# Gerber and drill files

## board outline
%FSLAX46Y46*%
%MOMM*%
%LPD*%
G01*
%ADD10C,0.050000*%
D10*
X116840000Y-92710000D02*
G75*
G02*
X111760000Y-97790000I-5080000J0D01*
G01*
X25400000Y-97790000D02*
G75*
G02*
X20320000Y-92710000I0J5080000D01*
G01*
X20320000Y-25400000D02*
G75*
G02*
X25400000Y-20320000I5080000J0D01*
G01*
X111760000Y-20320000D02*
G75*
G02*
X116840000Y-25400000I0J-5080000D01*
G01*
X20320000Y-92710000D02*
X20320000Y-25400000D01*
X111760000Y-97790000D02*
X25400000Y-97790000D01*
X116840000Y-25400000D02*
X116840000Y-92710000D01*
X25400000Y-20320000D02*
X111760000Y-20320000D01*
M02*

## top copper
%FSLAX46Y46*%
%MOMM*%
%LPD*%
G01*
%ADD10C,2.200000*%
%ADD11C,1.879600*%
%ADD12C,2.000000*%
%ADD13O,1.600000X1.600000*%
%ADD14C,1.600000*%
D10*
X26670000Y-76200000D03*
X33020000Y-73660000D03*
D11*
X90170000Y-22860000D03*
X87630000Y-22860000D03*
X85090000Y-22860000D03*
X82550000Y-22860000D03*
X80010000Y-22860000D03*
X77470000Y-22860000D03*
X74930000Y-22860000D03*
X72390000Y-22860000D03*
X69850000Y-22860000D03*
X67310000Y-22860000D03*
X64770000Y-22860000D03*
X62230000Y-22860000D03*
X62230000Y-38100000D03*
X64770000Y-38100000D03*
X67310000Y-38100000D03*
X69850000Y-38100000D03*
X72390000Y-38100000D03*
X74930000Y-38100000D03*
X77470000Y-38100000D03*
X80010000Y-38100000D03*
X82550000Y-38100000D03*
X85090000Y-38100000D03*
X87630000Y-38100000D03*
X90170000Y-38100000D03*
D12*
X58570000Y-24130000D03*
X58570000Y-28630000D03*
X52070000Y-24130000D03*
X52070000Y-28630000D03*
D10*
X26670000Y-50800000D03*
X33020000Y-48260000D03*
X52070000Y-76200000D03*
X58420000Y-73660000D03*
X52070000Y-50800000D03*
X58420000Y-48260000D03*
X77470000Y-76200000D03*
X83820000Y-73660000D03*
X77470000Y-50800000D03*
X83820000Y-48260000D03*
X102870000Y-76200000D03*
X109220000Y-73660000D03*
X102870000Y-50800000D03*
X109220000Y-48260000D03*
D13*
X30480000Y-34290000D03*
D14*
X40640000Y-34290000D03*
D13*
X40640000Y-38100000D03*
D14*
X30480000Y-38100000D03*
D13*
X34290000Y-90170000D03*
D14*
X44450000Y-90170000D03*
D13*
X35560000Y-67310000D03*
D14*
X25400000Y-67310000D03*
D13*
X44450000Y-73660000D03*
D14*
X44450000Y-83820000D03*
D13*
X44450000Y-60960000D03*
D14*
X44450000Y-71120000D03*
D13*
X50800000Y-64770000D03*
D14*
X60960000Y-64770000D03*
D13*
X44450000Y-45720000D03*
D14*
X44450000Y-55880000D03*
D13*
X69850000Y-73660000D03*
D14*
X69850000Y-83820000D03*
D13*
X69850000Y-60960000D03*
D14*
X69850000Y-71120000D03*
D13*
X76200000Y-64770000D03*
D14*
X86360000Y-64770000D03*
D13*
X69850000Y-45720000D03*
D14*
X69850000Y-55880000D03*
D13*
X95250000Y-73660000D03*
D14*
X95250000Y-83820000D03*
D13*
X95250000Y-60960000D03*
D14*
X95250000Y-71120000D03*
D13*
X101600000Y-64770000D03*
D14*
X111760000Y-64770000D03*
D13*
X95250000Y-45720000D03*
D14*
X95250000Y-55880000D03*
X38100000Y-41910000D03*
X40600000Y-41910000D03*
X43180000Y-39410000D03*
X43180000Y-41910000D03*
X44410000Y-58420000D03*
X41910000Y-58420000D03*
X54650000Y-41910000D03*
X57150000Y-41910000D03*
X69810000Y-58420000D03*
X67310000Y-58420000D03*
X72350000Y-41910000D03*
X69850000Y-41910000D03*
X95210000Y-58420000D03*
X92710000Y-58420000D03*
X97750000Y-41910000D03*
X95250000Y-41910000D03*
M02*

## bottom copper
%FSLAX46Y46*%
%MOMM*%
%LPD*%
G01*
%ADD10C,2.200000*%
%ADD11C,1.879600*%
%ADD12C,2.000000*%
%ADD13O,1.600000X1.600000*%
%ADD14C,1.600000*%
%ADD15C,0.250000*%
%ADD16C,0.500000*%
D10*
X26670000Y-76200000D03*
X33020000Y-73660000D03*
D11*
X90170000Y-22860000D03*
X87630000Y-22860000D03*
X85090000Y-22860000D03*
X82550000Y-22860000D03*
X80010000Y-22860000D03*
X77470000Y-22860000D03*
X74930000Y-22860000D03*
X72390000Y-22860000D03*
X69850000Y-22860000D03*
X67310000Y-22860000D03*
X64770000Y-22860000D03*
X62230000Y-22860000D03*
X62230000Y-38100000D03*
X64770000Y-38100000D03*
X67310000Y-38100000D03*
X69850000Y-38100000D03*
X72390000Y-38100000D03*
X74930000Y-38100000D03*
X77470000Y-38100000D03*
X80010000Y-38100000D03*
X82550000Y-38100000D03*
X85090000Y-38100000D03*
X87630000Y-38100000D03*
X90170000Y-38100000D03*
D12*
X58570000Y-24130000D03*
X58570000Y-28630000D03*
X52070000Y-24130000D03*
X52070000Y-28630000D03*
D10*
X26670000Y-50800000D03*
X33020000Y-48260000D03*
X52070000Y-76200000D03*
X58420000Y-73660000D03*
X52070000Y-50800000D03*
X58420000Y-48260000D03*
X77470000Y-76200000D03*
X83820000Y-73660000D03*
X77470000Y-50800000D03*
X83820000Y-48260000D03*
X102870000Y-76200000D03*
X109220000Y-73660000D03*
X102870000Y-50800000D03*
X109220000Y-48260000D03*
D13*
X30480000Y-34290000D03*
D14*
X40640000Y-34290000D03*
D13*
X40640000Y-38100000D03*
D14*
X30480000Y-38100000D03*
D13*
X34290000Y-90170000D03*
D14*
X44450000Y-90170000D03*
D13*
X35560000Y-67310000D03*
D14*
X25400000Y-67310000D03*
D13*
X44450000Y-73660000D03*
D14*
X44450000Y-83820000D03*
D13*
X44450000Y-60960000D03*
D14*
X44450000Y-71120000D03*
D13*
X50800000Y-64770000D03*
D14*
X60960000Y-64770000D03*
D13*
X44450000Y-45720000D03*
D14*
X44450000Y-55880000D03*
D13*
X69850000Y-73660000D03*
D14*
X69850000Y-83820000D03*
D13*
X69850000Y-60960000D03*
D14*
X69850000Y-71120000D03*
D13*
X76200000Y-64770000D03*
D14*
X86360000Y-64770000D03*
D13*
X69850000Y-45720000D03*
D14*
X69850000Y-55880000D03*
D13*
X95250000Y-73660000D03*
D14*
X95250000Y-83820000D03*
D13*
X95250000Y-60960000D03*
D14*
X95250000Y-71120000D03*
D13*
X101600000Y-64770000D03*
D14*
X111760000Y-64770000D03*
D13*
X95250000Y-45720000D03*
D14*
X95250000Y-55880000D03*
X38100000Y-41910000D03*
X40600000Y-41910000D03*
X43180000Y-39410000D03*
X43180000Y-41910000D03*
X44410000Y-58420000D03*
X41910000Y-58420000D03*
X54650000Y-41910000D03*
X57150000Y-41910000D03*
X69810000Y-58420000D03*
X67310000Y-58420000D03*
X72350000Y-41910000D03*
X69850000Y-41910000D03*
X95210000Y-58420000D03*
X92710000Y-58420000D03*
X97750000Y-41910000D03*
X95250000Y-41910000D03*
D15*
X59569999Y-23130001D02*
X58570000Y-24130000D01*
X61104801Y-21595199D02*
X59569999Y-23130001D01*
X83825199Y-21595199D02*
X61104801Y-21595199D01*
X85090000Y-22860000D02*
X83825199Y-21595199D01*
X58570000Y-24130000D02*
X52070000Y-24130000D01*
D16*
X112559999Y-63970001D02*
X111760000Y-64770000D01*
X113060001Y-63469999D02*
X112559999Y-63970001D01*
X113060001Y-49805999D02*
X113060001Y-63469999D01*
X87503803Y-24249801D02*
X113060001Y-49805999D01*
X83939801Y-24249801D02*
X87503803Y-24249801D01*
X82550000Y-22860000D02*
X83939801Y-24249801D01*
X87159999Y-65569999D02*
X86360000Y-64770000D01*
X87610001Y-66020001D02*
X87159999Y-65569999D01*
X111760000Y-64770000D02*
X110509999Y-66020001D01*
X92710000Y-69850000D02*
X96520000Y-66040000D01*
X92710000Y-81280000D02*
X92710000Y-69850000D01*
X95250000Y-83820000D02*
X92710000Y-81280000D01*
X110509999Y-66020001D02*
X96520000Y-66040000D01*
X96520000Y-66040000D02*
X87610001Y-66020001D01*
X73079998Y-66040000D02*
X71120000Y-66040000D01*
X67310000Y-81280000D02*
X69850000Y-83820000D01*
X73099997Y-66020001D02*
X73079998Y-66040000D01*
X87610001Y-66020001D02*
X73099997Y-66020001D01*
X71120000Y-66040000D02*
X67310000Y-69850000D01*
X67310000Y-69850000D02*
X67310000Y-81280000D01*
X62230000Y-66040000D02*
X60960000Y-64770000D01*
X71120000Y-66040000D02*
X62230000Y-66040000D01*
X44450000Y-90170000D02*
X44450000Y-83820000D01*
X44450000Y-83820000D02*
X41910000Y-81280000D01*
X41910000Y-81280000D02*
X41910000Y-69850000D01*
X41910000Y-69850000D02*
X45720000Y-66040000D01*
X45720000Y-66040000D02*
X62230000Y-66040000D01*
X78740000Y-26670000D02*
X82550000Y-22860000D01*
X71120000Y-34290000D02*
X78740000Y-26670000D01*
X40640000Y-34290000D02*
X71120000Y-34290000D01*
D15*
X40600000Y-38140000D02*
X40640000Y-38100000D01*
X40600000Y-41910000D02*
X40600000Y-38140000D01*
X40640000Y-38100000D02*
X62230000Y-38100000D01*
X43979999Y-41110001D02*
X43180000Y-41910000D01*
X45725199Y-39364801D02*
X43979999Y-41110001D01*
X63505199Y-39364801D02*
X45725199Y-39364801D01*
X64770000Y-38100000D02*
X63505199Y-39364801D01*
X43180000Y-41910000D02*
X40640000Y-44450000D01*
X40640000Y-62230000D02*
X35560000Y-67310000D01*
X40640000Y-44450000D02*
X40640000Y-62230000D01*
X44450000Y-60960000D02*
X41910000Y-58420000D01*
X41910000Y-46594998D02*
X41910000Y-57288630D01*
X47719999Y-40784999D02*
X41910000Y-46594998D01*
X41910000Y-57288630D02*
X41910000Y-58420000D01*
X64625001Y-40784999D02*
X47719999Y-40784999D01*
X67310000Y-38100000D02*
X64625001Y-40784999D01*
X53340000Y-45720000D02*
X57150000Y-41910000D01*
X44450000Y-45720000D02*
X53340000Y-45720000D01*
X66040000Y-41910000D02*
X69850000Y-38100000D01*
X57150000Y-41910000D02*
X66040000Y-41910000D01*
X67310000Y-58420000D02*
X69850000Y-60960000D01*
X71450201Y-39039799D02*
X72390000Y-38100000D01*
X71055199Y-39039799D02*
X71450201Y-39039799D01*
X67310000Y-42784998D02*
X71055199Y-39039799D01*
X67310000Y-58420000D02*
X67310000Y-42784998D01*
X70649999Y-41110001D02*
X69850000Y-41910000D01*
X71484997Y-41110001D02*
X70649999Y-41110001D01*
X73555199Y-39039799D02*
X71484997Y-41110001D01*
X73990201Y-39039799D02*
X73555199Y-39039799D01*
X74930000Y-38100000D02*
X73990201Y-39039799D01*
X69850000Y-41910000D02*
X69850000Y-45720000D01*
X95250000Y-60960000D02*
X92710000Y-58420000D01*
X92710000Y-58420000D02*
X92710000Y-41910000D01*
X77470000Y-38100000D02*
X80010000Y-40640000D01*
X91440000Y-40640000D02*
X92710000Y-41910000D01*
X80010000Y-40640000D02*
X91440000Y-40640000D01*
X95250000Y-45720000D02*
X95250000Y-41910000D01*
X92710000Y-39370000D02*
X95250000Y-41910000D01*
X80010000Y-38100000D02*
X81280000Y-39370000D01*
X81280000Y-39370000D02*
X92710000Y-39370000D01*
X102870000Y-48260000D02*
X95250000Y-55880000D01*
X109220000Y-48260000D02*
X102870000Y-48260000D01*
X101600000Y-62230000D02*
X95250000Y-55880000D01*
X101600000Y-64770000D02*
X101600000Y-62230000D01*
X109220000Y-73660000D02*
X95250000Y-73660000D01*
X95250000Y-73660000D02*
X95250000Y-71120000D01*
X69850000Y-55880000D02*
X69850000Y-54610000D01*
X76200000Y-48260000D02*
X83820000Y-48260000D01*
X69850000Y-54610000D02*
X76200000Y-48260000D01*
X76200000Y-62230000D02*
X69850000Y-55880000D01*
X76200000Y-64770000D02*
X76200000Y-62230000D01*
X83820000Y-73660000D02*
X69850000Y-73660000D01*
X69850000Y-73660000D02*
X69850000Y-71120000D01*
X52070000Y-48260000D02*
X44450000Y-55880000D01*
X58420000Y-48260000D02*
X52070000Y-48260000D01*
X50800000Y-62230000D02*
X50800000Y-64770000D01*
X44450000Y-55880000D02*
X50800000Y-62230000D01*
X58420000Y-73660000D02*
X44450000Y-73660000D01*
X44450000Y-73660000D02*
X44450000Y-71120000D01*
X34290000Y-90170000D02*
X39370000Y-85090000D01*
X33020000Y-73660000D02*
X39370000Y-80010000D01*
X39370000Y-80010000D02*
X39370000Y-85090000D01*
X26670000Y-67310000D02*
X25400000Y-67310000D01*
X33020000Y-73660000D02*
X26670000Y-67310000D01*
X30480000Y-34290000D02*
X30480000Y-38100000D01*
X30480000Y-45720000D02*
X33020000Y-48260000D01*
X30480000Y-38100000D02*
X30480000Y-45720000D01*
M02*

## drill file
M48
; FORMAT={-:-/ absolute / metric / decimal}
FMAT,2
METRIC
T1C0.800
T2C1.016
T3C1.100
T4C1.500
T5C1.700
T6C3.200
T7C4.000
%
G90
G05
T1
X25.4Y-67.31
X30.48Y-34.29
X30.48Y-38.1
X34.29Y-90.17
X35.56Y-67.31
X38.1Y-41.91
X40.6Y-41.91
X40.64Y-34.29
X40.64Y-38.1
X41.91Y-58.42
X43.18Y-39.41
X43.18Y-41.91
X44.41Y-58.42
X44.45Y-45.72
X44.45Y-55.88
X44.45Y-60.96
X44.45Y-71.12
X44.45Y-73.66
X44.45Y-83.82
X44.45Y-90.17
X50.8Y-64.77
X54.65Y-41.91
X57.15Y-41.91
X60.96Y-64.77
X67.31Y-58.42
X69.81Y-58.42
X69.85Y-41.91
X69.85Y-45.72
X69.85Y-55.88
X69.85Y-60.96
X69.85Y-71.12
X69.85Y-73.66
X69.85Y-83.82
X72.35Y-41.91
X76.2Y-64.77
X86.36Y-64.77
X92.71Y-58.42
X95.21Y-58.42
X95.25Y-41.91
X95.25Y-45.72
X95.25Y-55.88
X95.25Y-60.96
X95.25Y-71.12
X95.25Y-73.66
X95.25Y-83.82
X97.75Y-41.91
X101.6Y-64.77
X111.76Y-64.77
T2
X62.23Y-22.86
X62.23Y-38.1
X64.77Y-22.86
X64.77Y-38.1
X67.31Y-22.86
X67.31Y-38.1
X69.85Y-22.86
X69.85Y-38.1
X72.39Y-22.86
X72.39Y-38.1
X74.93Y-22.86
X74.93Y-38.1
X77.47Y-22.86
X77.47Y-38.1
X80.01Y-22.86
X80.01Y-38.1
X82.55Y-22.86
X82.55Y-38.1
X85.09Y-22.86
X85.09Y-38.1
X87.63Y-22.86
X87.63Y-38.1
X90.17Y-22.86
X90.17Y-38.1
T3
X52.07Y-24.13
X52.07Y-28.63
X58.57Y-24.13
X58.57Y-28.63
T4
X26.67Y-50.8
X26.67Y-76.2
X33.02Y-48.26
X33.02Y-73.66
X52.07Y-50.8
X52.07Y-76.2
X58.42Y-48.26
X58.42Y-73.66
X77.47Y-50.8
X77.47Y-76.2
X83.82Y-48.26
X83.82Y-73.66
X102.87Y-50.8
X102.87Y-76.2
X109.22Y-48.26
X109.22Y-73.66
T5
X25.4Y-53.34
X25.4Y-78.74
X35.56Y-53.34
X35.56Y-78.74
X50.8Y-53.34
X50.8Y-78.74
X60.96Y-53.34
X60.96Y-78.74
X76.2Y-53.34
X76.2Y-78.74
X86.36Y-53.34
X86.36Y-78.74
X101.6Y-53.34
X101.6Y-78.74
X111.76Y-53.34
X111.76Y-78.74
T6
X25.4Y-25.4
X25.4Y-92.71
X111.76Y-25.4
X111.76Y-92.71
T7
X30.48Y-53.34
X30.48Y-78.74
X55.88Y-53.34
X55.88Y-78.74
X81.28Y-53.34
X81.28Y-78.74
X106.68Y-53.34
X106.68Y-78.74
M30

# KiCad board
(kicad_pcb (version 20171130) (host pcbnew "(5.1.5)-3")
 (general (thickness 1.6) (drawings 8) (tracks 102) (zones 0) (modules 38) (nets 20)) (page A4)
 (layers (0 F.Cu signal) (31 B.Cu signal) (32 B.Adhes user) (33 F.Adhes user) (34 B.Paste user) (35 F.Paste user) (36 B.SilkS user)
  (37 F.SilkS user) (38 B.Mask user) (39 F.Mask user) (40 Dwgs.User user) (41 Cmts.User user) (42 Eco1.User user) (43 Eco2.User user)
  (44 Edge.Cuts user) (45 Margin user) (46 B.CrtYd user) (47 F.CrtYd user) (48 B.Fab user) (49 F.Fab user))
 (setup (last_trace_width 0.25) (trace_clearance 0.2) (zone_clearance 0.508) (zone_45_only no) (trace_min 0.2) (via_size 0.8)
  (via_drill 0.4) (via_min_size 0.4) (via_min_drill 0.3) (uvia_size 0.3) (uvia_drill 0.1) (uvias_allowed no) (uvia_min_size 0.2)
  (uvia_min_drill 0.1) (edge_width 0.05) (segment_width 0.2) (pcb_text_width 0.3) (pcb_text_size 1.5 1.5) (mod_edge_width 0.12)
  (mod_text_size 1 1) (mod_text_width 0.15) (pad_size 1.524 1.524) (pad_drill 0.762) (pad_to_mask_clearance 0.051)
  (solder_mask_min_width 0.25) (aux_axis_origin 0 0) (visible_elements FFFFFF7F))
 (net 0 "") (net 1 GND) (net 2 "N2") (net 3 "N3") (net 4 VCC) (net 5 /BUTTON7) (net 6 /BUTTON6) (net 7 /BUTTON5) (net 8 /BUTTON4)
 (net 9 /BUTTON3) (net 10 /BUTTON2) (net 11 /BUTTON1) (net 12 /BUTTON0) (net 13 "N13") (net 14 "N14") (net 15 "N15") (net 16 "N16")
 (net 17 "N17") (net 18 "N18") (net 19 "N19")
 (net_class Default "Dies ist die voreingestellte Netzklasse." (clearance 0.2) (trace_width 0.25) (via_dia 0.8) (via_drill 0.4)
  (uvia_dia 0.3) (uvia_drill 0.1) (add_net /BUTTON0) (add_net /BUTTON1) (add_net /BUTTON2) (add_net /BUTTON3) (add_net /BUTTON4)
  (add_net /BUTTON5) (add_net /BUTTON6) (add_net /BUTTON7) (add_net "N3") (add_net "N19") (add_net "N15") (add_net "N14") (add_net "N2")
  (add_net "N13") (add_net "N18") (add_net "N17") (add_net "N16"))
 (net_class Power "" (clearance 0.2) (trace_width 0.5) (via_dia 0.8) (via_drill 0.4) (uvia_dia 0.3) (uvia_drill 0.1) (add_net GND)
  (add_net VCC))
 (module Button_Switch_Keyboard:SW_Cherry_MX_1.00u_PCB (layer F.Cu) (at 33.02 73.66)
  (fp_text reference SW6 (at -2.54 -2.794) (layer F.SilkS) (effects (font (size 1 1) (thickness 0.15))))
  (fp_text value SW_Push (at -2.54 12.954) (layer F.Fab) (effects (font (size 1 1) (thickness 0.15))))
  (pad "" np_thru_hole circle (at 2.54 5.08) (size 1.7 1.7) (drill 1.7) (layers *.Cu *.Mask))
  (pad "" np_thru_hole circle (at -7.62 5.08) (size 1.7 1.7) (drill 1.7) (layers *.Cu *.Mask))
  (pad "" np_thru_hole circle (at -2.54 5.08) (size 4 4) (drill 4) (layers *.Cu *.Mask))
  (pad 2 thru_hole circle (at -6.35 2.54) (size 2.2 2.2) (drill 1.5) (layers *.Cu *.Mask) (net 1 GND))
  (pad 1 thru_hole circle (at 0 0) (size 2.2 2.2) (drill 1.5) (layers *.Cu *.Mask) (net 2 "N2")))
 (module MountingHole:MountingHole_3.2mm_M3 (layer F.Cu) (at 25.4 25.4)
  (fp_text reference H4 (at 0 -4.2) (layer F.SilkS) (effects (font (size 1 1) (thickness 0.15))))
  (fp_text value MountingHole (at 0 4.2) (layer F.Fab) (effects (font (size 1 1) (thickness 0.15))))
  (pad 1 np_thru_hole circle (at 0 0) (size 3.2 3.2) (drill 3.2) (layers *.Cu *.Mask)))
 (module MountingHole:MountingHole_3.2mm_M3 (layer F.Cu) (at 111.76 25.4)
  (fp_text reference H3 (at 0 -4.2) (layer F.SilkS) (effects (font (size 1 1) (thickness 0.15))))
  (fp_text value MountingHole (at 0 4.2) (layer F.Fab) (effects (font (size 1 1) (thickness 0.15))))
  (pad 1 np_thru_hole circle (at 0 0) (size 3.2 3.2) (drill 3.2) (layers *.Cu *.Mask)))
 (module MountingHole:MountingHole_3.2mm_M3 (layer F.Cu) (at 111.76 92.71)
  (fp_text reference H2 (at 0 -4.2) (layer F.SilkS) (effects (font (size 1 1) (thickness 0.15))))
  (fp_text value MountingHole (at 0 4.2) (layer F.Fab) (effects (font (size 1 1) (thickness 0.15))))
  (pad 1 np_thru_hole circle (at 0 0) (size 3.2 3.2) (drill 3.2) (layers *.Cu *.Mask)))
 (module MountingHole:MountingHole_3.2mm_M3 (layer F.Cu) (at 25.4 92.71)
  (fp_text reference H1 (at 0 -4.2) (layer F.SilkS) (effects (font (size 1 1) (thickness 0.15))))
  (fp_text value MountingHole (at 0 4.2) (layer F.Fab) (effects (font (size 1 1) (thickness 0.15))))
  (pad 1 np_thru_hole circle (at 0 0) (size 3.2 3.2) (drill 3.2) (layers *.Cu *.Mask)))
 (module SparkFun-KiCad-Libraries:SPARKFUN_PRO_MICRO (layer B.Cu) (at 77.47 30.48 90)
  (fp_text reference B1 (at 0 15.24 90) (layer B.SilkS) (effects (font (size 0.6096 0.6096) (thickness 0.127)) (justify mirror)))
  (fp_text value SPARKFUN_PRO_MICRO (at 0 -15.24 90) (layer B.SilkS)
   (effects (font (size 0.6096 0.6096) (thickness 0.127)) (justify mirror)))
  (pad 24 thru_hole circle (at 7.62 12.7 90) (size 1.8796 1.8796) (drill 1.016) (layers *.Cu *.Mask) (solder_mask_margin 0.1016))
  (pad 23 thru_hole circle (at 7.62 10.16 90) (size 1.8796 1.8796) (drill 1.016) (layers *.Cu *.Mask) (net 1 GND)
   (solder_mask_margin 0.1016))
  (pad 22 thru_hole circle (at 7.62 7.62 90) (size 1.8796 1.8796) (drill 1.016) (layers *.Cu *.Mask) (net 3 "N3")
   (solder_mask_margin 0.1016))
  (pad 21 thru_hole circle (at 7.62 5.08 90) (size 1.8796 1.8796) (drill 1.016) (layers *.Cu *.Mask) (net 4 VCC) (solder_mask_margin 0.1016))
  (pad 20 thru_hole circle (at 7.62 2.54 90) (size 1.8796 1.8796) (drill 1.016) (layers *.Cu *.Mask) (solder_mask_margin 0.1016))
  (pad 19 thru_hole circle (at 7.62 0 90) (size 1.8796 1.8796) (drill 1.016) (layers *.Cu *.Mask) (solder_mask_margin 0.1016))
  (pad 18 thru_hole circle (at 7.62 -2.54 90) (size 1.8796 1.8796) (drill 1.016) (layers *.Cu *.Mask) (solder_mask_margin 0.1016))
  (pad 17 thru_hole circle (at 7.62 -5.08 90) (size 1.8796 1.8796) (drill 1.016) (layers *.Cu *.Mask) (solder_mask_margin 0.1016))
  (pad 16 thru_hole circle (at 7.62 -7.62 90) (size 1.8796 1.8796) (drill 1.016) (layers *.Cu *.Mask) (solder_mask_margin 0.1016))
  (pad 15 thru_hole circle (at 7.62 -10.16 90) (size 1.8796 1.8796) (drill 1.016) (layers *.Cu *.Mask) (solder_mask_margin 0.1016))
  (pad 14 thru_hole circle (at 7.62 -12.7 90) (size 1.8796 1.8796) (drill 1.016) (layers *.Cu *.Mask) (solder_mask_margin 0.1016))
  (pad 13 thru_hole circle (at 7.62 -15.24 90) (size 1.8796 1.8796) (drill 1.016) (layers *.Cu *.Mask) (solder_mask_margin 0.1016))
  (pad 12 thru_hole circle (at -7.62 -15.24 90) (size 1.8796 1.8796) (drill 1.016) (layers *.Cu *.Mask) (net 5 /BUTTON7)
   (solder_mask_margin 0.1016))
  (pad 11 thru_hole circle (at -7.62 -12.7 90) (size 1.8796 1.8796) (drill 1.016) (layers *.Cu *.Mask) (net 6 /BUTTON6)
   (solder_mask_margin 0.1016))
  (pad 10 thru_hole circle (at -7.62 -10.16 90) (size 1.8796 1.8796) (drill 1.016) (layers *.Cu *.Mask) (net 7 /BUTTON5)
   (solder_mask_margin 0.1016))
  (pad 9 thru_hole circle (at -7.62 -7.62 90) (size 1.8796 1.8796) (drill 1.016) (layers *.Cu *.Mask) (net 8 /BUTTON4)
   (solder_mask_margin 0.1016))
  (pad 8 thru_hole circle (at -7.62 -5.08 90) (size 1.8796 1.8796) (drill 1.016) (layers *.Cu *.Mask) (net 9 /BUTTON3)
   (solder_mask_margin 0.1016))
  (pad 7 thru_hole circle (at -7.62 -2.54 90) (size 1.8796 1.8796) (drill 1.016) (layers *.Cu *.Mask) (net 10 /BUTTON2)
   (solder_mask_margin 0.1016))
  (pad 6 thru_hole circle (at -7.62 0 90) (size 1.8796 1.8796) (drill 1.016) (layers *.Cu *.Mask) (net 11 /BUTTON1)
   (solder_mask_margin 0.1016))
  (pad 5 thru_hole circle (at -7.62 2.54 90) (size 1.8796 1.8796) (drill 1.016) (layers *.Cu *.Mask) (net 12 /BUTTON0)
   (solder_mask_margin 0.1016))
  (pad 4 thru_hole circle (at -7.62 5.08 90) (size 1.8796 1.8796) (drill 1.016) (layers *.Cu *.Mask) (solder_mask_margin 0.1016))
  (pad 3 thru_hole circle (at -7.62 7.62 90) (size 1.8796 1.8796) (drill 1.016) (layers *.Cu *.Mask) (solder_mask_margin 0.1016))
  (pad 2 thru_hole circle (at -7.62 10.16 90) (size 1.8796 1.8796) (drill 1.016) (layers *.Cu *.Mask) (solder_mask_margin 0.1016))
  (pad 1 thru_hole circle (at -7.62 12.7 90) (size 1.8796 1.8796) (drill 1.016) (layers *.Cu *.Mask) (solder_mask_margin 0.1016)))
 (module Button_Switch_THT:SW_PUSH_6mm (layer F.Cu) (at 52.07 24.13)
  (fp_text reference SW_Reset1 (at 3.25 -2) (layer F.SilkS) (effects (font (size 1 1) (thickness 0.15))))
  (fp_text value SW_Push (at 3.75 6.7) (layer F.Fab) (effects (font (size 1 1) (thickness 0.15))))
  (pad 1 thru_hole circle (at 6.5 0 90) (size 2 2) (drill 1.1) (layers *.Cu *.Mask) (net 3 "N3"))
  (pad 2 thru_hole circle (at 6.5 4.5 90) (size 2 2) (drill 1.1) (layers *.Cu *.Mask) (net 1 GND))
  (pad 1 thru_hole circle (at 0 0 90) (size 2 2) (drill 1.1) (layers *.Cu *.Mask) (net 3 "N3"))
  (pad 2 thru_hole circle (at 0 4.5 90) (size 2 2) (drill 1.1) (layers *.Cu *.Mask) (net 1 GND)))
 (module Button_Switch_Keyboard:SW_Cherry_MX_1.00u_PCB (layer F.Cu) (at 33.02 48.26)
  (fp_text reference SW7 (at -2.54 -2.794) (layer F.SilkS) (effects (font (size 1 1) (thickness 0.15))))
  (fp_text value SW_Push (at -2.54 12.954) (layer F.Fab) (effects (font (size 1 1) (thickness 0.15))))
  (pad "" np_thru_hole circle (at 2.54 5.08) (size 1.7 1.7) (drill 1.7) (layers *.Cu *.Mask))
  (pad "" np_thru_hole circle (at -7.62 5.08) (size 1.7 1.7) (drill 1.7) (layers *.Cu *.Mask))
  (pad "" np_thru_hole circle (at -2.54 5.08) (size 4 4) (drill 4) (layers *.Cu *.Mask))
  (pad 2 thru_hole circle (at -6.35 2.54) (size 2.2 2.2) (drill 1.5) (layers *.Cu *.Mask) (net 1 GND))
  (pad 1 thru_hole circle (at 0 0) (size 2.2 2.2) (drill 1.5) (layers *.Cu *.Mask) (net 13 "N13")))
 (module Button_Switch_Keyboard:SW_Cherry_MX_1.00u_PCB (layer F.Cu) (at 58.42 73.66)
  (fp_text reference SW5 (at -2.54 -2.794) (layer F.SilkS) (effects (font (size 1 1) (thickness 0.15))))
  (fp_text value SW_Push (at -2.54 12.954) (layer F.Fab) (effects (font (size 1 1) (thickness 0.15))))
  (pad "" np_thru_hole circle (at 2.54 5.08) (size 1.7 1.7) (drill 1.7) (layers *.Cu *.Mask))
  (pad "" np_thru_hole circle (at -7.62 5.08) (size 1.7 1.7) (drill 1.7) (layers *.Cu *.Mask))
  (pad "" np_thru_hole circle (at -2.54 5.08) (size 4 4) (drill 4) (layers *.Cu *.Mask))
  (pad 2 thru_hole circle (at -6.35 2.54) (size 2.2 2.2) (drill 1.5) (layers *.Cu *.Mask) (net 1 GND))
  (pad 1 thru_hole circle (at 0 0) (size 2.2 2.2) (drill 1.5) (layers *.Cu *.Mask) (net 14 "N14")))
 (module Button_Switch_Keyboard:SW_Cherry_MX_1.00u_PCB (layer F.Cu) (at 58.42 48.26)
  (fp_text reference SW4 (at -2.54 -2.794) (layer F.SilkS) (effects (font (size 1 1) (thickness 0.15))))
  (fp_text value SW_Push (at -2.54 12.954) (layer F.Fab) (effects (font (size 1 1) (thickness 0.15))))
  (pad "" np_thru_hole circle (at 2.54 5.08) (size 1.7 1.7) (drill 1.7) (layers *.Cu *.Mask))
  (pad "" np_thru_hole circle (at -7.62 5.08) (size 1.7 1.7) (drill 1.7) (layers *.Cu *.Mask))
  (pad "" np_thru_hole circle (at -2.54 5.08) (size 4 4) (drill 4) (layers *.Cu *.Mask))
  (pad 2 thru_hole circle (at -6.35 2.54) (size 2.2 2.2) (drill 1.5) (layers *.Cu *.Mask) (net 1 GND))
  (pad 1 thru_hole circle (at 0 0) (size 2.2 2.2) (drill 1.5) (layers *.Cu *.Mask) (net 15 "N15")))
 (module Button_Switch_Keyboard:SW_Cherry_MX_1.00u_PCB (layer F.Cu) (at 83.82 73.66)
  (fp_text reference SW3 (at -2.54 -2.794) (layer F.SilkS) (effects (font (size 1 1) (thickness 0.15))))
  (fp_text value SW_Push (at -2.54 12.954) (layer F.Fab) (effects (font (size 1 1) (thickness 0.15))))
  (pad "" np_thru_hole circle (at 2.54 5.08) (size 1.7 1.7) (drill 1.7) (layers *.Cu *.Mask))
  (pad "" np_thru_hole circle (at -7.62 5.08) (size 1.7 1.7) (drill 1.7) (layers *.Cu *.Mask))
  (pad "" np_thru_hole circle (at -2.54 5.08) (size 4 4) (drill 4) (layers *.Cu *.Mask))
  (pad 2 thru_hole circle (at -6.35 2.54) (size 2.2 2.2) (drill 1.5) (layers *.Cu *.Mask) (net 1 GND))
  (pad 1 thru_hole circle (at 0 0) (size 2.2 2.2) (drill 1.5) (layers *.Cu *.Mask) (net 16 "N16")))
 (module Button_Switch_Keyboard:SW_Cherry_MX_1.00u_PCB (layer F.Cu) (at 83.82 48.26)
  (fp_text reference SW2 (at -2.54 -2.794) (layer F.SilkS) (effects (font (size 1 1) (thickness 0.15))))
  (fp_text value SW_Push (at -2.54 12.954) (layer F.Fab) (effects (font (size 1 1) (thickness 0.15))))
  (pad "" np_thru_hole circle (at 2.54 5.08) (size 1.7 1.7) (drill 1.7) (layers *.Cu *.Mask))
  (pad "" np_thru_hole circle (at -7.62 5.08) (size 1.7 1.7) (drill 1.7) (layers *.Cu *.Mask))
  (pad "" np_thru_hole circle (at -2.54 5.08) (size 4 4) (drill 4) (layers *.Cu *.Mask))
  (pad 2 thru_hole circle (at -6.35 2.54) (size 2.2 2.2) (drill 1.5) (layers *.Cu *.Mask) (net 1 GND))
  (pad 1 thru_hole circle (at 0 0) (size 2.2 2.2) (drill 1.5) (layers *.Cu *.Mask) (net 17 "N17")))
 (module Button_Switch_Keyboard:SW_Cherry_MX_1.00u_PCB (layer F.Cu) (at 109.22 73.66)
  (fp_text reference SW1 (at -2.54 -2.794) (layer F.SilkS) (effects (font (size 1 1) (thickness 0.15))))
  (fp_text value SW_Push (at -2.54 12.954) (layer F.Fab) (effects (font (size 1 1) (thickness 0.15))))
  (pad "" np_thru_hole circle (at 2.54 5.08) (size 1.7 1.7) (drill 1.7) (layers *.Cu *.Mask))
  (pad "" np_thru_hole circle (at -7.62 5.08) (size 1.7 1.7) (drill 1.7) (layers *.Cu *.Mask))
  (pad "" np_thru_hole circle (at -2.54 5.08) (size 4 4) (drill 4) (layers *.Cu *.Mask))
  (pad 2 thru_hole circle (at -6.35 2.54) (size 2.2 2.2) (drill 1.5) (layers *.Cu *.Mask) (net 1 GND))
  (pad 1 thru_hole circle (at 0 0) (size 2.2 2.2) (drill 1.5) (layers *.Cu *.Mask) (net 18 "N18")))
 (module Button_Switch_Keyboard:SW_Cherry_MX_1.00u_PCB (layer F.Cu) (at 109.22 48.26)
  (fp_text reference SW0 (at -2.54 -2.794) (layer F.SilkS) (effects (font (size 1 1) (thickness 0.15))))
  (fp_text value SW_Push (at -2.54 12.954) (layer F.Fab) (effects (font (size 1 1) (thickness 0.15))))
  (pad "" np_thru_hole circle (at 2.54 5.08) (size 1.7 1.7) (drill 1.7) (layers *.Cu *.Mask))
  (pad "" np_thru_hole circle (at -7.62 5.08) (size 1.7 1.7) (drill 1.7) (layers *.Cu *.Mask))
  (pad "" np_thru_hole circle (at -2.54 5.08) (size 4 4) (drill 4) (layers *.Cu *.Mask))
  (pad 2 thru_hole circle (at -6.35 2.54) (size 2.2 2.2) (drill 1.5) (layers *.Cu *.Mask) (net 1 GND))
  (pad 1 thru_hole circle (at 0 0) (size 2.2 2.2) (drill 1.5) (layers *.Cu *.Mask) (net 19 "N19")))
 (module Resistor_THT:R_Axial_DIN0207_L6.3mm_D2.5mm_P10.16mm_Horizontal (layer F.Cu) (at 40.64 34.29 180)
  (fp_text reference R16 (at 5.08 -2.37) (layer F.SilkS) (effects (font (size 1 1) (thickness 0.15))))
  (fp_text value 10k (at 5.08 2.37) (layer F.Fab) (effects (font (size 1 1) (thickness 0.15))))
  (pad 2 thru_hole oval (at 10.16 0 180) (size 1.6 1.6) (drill 0.8) (layers *.Cu *.Mask) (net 13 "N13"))
  (pad 1 thru_hole circle (at 0 0 180) (size 1.6 1.6) (drill 0.8) (layers *.Cu *.Mask) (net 4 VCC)))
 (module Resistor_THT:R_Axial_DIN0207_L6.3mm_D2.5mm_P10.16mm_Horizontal (layer F.Cu) (at 30.48 38.1)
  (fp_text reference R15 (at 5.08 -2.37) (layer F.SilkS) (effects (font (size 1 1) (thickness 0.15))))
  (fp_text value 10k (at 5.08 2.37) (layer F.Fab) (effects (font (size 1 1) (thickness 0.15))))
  (pad 2 thru_hole oval (at 10.16 0) (size 1.6 1.6) (drill 0.8) (layers *.Cu *.Mask) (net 5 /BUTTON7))
  (pad 1 thru_hole circle (at 0 0) (size 1.6 1.6) (drill 0.8) (layers *.Cu *.Mask) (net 13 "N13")))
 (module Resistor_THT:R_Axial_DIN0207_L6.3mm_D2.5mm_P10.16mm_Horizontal (layer F.Cu) (at 44.45 90.17 180)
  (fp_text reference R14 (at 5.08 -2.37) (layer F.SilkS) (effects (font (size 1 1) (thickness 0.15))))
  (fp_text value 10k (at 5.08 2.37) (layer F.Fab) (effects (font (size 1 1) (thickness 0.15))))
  (pad 2 thru_hole oval (at 10.16 0 180) (size 1.6 1.6) (drill 0.8) (layers *.Cu *.Mask) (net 2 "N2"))
  (pad 1 thru_hole circle (at 0 0 180) (size 1.6 1.6) (drill 0.8) (layers *.Cu *.Mask) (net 4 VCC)))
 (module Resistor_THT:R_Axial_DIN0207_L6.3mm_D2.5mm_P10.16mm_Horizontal (layer F.Cu) (at 25.4 67.31)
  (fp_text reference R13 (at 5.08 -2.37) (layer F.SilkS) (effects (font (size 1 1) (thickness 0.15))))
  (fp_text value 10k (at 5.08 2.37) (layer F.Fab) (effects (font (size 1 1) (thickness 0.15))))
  (pad 2 thru_hole oval (at 10.16 0) (size 1.6 1.6) (drill 0.8) (layers *.Cu *.Mask) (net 6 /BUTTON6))
  (pad 1 thru_hole circle (at 0 0) (size 1.6 1.6) (drill 0.8) (layers *.Cu *.Mask) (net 2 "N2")))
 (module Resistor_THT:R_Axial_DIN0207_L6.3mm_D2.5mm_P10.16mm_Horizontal (layer F.Cu) (at 44.45 83.82 90)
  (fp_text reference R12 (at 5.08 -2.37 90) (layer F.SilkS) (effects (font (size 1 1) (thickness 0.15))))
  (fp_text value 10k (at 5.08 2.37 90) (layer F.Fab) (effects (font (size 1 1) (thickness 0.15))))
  (pad 2 thru_hole oval (at 10.16 0 90) (size 1.6 1.6) (drill 0.8) (layers *.Cu *.Mask) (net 14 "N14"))
  (pad 1 thru_hole circle (at 0 0 90) (size 1.6 1.6) (drill 0.8) (layers *.Cu *.Mask) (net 4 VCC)))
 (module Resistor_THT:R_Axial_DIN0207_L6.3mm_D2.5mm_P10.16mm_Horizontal (layer F.Cu) (at 44.45 71.12 90)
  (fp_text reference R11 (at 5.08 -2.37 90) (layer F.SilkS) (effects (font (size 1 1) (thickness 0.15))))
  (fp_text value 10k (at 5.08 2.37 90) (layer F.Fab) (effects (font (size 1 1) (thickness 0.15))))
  (pad 2 thru_hole oval (at 10.16 0 90) (size 1.6 1.6) (drill 0.8) (layers *.Cu *.Mask) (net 7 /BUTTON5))
  (pad 1 thru_hole circle (at 0 0 90) (size 1.6 1.6) (drill 0.8) (layers *.Cu *.Mask) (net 14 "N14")))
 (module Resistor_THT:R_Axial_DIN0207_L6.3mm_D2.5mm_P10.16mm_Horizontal (layer F.Cu) (at 60.96 64.77 180)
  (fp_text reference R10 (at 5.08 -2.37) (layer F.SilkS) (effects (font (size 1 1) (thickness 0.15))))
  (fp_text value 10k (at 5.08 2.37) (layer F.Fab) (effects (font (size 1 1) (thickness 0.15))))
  (pad 2 thru_hole oval (at 10.16 0 180) (size 1.6 1.6) (drill 0.8) (layers *.Cu *.Mask) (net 15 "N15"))
  (pad 1 thru_hole circle (at 0 0 180) (size 1.6 1.6) (drill 0.8) (layers *.Cu *.Mask) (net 4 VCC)))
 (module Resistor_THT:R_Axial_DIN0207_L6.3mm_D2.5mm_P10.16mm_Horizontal (layer F.Cu) (at 44.45 55.88 90)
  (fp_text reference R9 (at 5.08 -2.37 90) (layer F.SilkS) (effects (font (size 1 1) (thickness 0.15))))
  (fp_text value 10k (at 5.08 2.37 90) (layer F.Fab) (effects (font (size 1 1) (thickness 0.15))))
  (pad 2 thru_hole oval (at 10.16 0 90) (size 1.6 1.6) (drill 0.8) (layers *.Cu *.Mask) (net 8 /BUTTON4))
  (pad 1 thru_hole circle (at 0 0 90) (size 1.6 1.6) (drill 0.8) (layers *.Cu *.Mask) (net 15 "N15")))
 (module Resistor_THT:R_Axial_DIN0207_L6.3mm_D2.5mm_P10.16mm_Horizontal (layer F.Cu) (at 69.85 83.82 90)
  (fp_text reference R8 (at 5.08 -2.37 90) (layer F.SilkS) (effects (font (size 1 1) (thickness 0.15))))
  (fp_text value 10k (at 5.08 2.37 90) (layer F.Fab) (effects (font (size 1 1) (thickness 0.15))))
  (pad 2 thru_hole oval (at 10.16 0 90) (size 1.6 1.6) (drill 0.8) (layers *.Cu *.Mask) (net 16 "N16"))
  (pad 1 thru_hole circle (at 0 0 90) (size 1.6 1.6) (drill 0.8) (layers *.Cu *.Mask) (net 4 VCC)))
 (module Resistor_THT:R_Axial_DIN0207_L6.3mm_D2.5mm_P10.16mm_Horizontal (layer F.Cu) (at 69.85 71.12 90)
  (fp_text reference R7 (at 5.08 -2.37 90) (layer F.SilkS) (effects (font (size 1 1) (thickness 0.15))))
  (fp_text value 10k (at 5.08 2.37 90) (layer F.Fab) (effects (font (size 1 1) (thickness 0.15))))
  (pad 2 thru_hole oval (at 10.16 0 90) (size 1.6 1.6) (drill 0.8) (layers *.Cu *.Mask) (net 9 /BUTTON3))
  (pad 1 thru_hole circle (at 0 0 90) (size 1.6 1.6) (drill 0.8) (layers *.Cu *.Mask) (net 16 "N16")))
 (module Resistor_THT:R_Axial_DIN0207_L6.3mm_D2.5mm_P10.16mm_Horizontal (layer F.Cu) (at 86.36 64.77 180)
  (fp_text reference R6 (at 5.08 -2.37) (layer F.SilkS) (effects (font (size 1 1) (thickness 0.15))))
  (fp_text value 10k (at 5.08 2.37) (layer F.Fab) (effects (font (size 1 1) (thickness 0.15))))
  (pad 2 thru_hole oval (at 10.16 0 180) (size 1.6 1.6) (drill 0.8) (layers *.Cu *.Mask) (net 17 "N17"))
  (pad 1 thru_hole circle (at 0 0 180) (size 1.6 1.6) (drill 0.8) (layers *.Cu *.Mask) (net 4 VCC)))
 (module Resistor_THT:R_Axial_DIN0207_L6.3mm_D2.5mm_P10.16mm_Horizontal (layer F.Cu) (at 69.85 55.88 90)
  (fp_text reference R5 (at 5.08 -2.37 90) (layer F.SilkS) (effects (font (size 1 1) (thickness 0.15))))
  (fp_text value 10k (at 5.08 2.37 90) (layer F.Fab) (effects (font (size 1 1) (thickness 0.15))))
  (pad 2 thru_hole oval (at 10.16 0 90) (size 1.6 1.6) (drill 0.8) (layers *.Cu *.Mask) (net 10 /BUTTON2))
  (pad 1 thru_hole circle (at 0 0 90) (size 1.6 1.6) (drill 0.8) (layers *.Cu *.Mask) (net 17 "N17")))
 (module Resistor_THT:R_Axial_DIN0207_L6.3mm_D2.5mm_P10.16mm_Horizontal (layer F.Cu) (at 95.25 83.82 90)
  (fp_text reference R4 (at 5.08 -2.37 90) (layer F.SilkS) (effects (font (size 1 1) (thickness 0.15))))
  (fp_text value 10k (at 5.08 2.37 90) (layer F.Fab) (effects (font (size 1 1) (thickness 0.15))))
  (pad 2 thru_hole oval (at 10.16 0 90) (size 1.6 1.6) (drill 0.8) (layers *.Cu *.Mask) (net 18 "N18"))
  (pad 1 thru_hole circle (at 0 0 90) (size 1.6 1.6) (drill 0.8) (layers *.Cu *.Mask) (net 4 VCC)))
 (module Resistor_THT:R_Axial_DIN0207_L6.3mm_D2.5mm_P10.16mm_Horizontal (layer F.Cu) (at 95.25 71.12 90)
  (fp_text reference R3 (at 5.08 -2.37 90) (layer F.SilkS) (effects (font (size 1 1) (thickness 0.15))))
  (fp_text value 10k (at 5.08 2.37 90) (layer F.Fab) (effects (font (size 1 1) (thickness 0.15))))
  (pad 2 thru_hole oval (at 10.16 0 90) (size 1.6 1.6) (drill 0.8) (layers *.Cu *.Mask) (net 11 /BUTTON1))
  (pad 1 thru_hole circle (at 0 0 90) (size 1.6 1.6) (drill 0.8) (layers *.Cu *.Mask) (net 18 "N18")))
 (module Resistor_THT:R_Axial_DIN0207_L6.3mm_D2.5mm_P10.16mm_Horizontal (layer F.Cu) (at 111.76 64.77 180)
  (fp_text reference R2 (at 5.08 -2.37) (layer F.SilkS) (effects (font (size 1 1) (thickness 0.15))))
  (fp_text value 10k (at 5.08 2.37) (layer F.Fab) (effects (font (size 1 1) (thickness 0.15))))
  (pad 2 thru_hole oval (at 10.16 0 180) (size 1.6 1.6) (drill 0.8) (layers *.Cu *.Mask) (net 19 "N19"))
  (pad 1 thru_hole circle (at 0 0 180) (size 1.6 1.6) (drill 0.8) (layers *.Cu *.Mask) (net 4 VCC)))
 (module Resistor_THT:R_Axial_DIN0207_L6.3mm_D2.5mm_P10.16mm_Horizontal (layer F.Cu) (at 95.25 55.88 90)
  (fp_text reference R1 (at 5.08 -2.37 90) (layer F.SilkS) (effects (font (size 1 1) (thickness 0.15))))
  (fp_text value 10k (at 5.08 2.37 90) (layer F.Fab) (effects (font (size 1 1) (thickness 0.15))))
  (pad 2 thru_hole oval (at 10.16 0 90) (size 1.6 1.6) (drill 0.8) (layers *.Cu *.Mask) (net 12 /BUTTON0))
  (pad 1 thru_hole circle (at 0 0 90) (size 1.6 1.6) (drill 0.8) (layers *.Cu *.Mask) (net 19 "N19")))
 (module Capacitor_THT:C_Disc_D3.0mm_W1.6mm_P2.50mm (layer F.Cu) (at 40.6 41.91 180)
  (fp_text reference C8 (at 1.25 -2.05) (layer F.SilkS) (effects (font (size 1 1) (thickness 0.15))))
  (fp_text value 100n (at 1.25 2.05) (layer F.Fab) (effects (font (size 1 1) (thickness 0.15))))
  (pad 2 thru_hole circle (at 2.5 0 180) (size 1.6 1.6) (drill 0.8) (layers *.Cu *.Mask) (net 1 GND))
  (pad 1 thru_hole circle (at 0 0 180) (size 1.6 1.6) (drill 0.8) (layers *.Cu *.Mask) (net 5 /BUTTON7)))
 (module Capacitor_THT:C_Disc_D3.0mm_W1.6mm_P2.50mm (layer F.Cu) (at 43.18 41.91 90)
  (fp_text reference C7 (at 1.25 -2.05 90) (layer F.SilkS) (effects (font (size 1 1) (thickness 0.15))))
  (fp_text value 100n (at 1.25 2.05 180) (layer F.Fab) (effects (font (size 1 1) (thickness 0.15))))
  (pad 2 thru_hole circle (at 2.5 0 90) (size 1.6 1.6) (drill 0.8) (layers *.Cu *.Mask) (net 1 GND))
  (pad 1 thru_hole circle (at 0 0 90) (size 1.6 1.6) (drill 0.8) (layers *.Cu *.Mask) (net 6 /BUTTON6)))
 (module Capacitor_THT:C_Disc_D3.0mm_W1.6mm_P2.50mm (layer F.Cu) (at 41.91 58.42)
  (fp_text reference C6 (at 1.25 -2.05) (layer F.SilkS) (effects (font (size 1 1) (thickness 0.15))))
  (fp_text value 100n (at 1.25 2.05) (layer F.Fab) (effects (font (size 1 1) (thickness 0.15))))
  (pad 2 thru_hole circle (at 2.5 0) (size 1.6 1.6) (drill 0.8) (layers *.Cu *.Mask) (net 1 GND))
  (pad 1 thru_hole circle (at 0 0) (size 1.6 1.6) (drill 0.8) (layers *.Cu *.Mask) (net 7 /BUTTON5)))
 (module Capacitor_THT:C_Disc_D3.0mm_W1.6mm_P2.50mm (layer F.Cu) (at 57.15 41.91 180)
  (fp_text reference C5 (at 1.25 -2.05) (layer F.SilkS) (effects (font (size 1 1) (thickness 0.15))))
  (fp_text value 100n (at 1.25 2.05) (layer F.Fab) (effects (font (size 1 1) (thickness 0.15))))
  (pad 2 thru_hole circle (at 2.5 0 180) (size 1.6 1.6) (drill 0.8) (layers *.Cu *.Mask) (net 1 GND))
  (pad 1 thru_hole circle (at 0 0 180) (size 1.6 1.6) (drill 0.8) (layers *.Cu *.Mask) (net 8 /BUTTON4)))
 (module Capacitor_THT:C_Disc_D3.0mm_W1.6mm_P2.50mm (layer F.Cu) (at 67.31 58.42)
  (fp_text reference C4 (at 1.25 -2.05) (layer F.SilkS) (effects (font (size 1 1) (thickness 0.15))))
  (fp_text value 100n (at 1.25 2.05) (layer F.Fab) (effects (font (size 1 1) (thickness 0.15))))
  (pad 2 thru_hole circle (at 2.5 0) (size 1.6 1.6) (drill 0.8) (layers *.Cu *.Mask) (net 1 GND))
  (pad 1 thru_hole circle (at 0 0) (size 1.6 1.6) (drill 0.8) (layers *.Cu *.Mask) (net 9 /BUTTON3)))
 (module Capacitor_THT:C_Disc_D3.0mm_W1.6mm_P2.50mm (layer F.Cu) (at 69.85 41.91)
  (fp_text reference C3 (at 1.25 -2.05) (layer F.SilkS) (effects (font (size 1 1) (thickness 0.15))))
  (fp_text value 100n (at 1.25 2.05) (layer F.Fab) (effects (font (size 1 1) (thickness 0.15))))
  (pad 2 thru_hole circle (at 2.5 0) (size 1.6 1.6) (drill 0.8) (layers *.Cu *.Mask) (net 1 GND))
  (pad 1 thru_hole circle (at 0 0) (size 1.6 1.6) (drill 0.8) (layers *.Cu *.Mask) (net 10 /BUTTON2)))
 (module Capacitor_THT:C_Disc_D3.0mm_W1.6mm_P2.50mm (layer F.Cu) (at 92.71 58.42)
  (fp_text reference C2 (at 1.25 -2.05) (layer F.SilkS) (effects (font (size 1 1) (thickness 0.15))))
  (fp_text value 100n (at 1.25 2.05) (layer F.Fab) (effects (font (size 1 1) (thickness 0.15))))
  (pad 2 thru_hole circle (at 2.5 0) (size 1.6 1.6) (drill 0.8) (layers *.Cu *.Mask) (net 1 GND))
  (pad 1 thru_hole circle (at 0 0) (size 1.6 1.6) (drill 0.8) (layers *.Cu *.Mask) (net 11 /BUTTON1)))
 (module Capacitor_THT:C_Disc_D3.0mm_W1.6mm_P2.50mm (layer F.Cu) (at 95.25 41.91)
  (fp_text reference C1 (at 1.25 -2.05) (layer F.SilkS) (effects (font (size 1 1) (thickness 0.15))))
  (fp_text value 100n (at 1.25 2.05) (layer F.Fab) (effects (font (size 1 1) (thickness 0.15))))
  (pad 2 thru_hole circle (at 2.5 0) (size 1.6 1.6) (drill 0.8) (layers *.Cu *.Mask) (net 1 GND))
  (pad 1 thru_hole circle (at 0 0) (size 1.6 1.6) (drill 0.8) (layers *.Cu *.Mask) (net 12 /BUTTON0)))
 (gr_arc (start 111.76 92.71) (end 111.76 97.79) (angle -90) (layer Edge.Cuts) (width 0.05))
 (gr_arc (start 25.4 92.71) (end 20.32 92.71) (angle -90) (layer Edge.Cuts) (width 0.05))
 (gr_arc (start 25.4 25.4) (end 25.4 20.32) (angle -90) (layer Edge.Cuts) (width 0.05))
 (gr_arc (start 111.76 25.4) (end 116.84 25.4) (angle -90) (layer Edge.Cuts) (width 0.05))
 (gr_line (start 20.32 92.71) (end 20.32 25.4) (layer Edge.Cuts) (width 0.05))
 (gr_line (start 111.76 97.79) (end 25.4 97.79) (layer Edge.Cuts) (width 0.05))
 (gr_line (start 116.84 25.4) (end 116.84 92.71) (layer Edge.Cuts) (width 0.05))
 (gr_line (start 25.4 20.32) (end 111.76 20.32) (layer Edge.Cuts) (width 0.05))
 (segment (start 59.569999 23.130001) (end 58.57 24.13) (width 0.25) (layer B.Cu) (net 3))
 (segment (start 61.104801 21.595199) (end 59.569999 23.130001) (width 0.25) (layer B.Cu) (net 3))
 (segment (start 83.825199 21.595199) (end 61.104801 21.595199) (width 0.25) (layer B.Cu) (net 3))
 (segment (start 85.09 22.86) (end 83.825199 21.595199) (width 0.25) (layer B.Cu) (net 3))
 (segment (start 58.57 24.13) (end 52.07 24.13) (width 0.25) (layer B.Cu) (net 3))
 (segment (start 112.559999 63.970001) (end 111.76 64.77) (width 0.5) (layer B.Cu) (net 4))
 (segment (start 113.060001 63.469999) (end 112.559999 63.970001) (width 0.5) (layer B.Cu) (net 4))
 (segment (start 113.060001 49.805999) (end 113.060001 63.469999) (width 0.5) (layer B.Cu) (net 4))
 (segment (start 87.503803 24.249801) (end 113.060001 49.805999) (width 0.5) (layer B.Cu) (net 4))
 (segment (start 83.939801 24.249801) (end 87.503803 24.249801) (width 0.5) (layer B.Cu) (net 4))
 (segment (start 82.55 22.86) (end 83.939801 24.249801) (width 0.5) (layer B.Cu) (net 4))
 (segment (start 87.159999 65.569999) (end 86.36 64.77) (width 0.5) (layer B.Cu) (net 4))
 (segment (start 87.610001 66.020001) (end 87.159999 65.569999) (width 0.5) (layer B.Cu) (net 4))
 (segment (start 111.76 64.77) (end 110.509999 66.020001) (width 0.5) (layer B.Cu) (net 4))
 (segment (start 92.71 69.85) (end 96.52 66.04) (width 0.5) (layer B.Cu) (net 4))
 (segment (start 92.71 81.28) (end 92.71 69.85) (width 0.5) (layer B.Cu) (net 4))
 (segment (start 95.25 83.82) (end 92.71 81.28) (width 0.5) (layer B.Cu) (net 4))
 (segment (start 110.509999 66.020001) (end 96.52 66.04) (width 0.5) (layer B.Cu) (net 4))
 (segment (start 96.52 66.04) (end 87.610001 66.020001) (width 0.5) (layer B.Cu) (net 4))
 (segment (start 73.079998 66.04) (end 71.12 66.04) (width 0.5) (layer B.Cu) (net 4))
 (segment (start 67.31 81.28) (end 69.85 83.82) (width 0.5) (layer B.Cu) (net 4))
 (segment (start 73.099997 66.020001) (end 73.079998 66.04) (width 0.5) (layer B.Cu) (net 4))
 (segment (start 87.610001 66.020001) (end 73.099997 66.020001) (width 0.5) (layer B.Cu) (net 4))
 (segment (start 71.12 66.04) (end 67.31 69.85) (width 0.5) (layer B.Cu) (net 4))
 (segment (start 67.31 69.85) (end 67.31 81.28) (width 0.5) (layer B.Cu) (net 4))
 (segment (start 62.23 66.04) (end 60.96 64.77) (width 0.5) (layer B.Cu) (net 4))
 (segment (start 71.12 66.04) (end 62.23 66.04) (width 0.5) (layer B.Cu) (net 4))
 (segment (start 44.45 90.17) (end 44.45 83.82) (width 0.5) (layer B.Cu) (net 4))
 (segment (start 44.45 83.82) (end 41.91 81.28) (width 0.5) (layer B.Cu) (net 4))
 (segment (start 41.91 81.28) (end 41.91 69.85) (width 0.5) (layer B.Cu) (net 4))
 (segment (start 41.91 69.85) (end 45.72 66.04) (width 0.5) (layer B.Cu) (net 4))
 (segment (start 45.72 66.04) (end 62.23 66.04) (width 0.5) (layer B.Cu) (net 4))
 (segment (start 78.74 26.67) (end 82.55 22.86) (width 0.5) (layer B.Cu) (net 4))
 (segment (start 71.12 34.29) (end 78.74 26.67) (width 0.5) (layer B.Cu) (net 4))
 (segment (start 40.64 34.29) (end 71.12 34.29) (width 0.5) (layer B.Cu) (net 4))
 (segment (start 40.6 38.14) (end 40.64 38.1) (width 0.25) (layer B.Cu) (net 5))
 (segment (start 40.6 41.91) (end 40.6 38.14) (width 0.25) (layer B.Cu) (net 5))
 (segment (start 40.64 38.1) (end 62.23 38.1) (width 0.25) (layer B.Cu) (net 5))
 (segment (start 43.979999 41.110001) (end 43.18 41.91) (width 0.25) (layer B.Cu) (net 6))
 (segment (start 45.725199 39.364801) (end 43.979999 41.110001) (width 0.25) (layer B.Cu) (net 6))
 (segment (start 63.505199 39.364801) (end 45.725199 39.364801) (width 0.25) (layer B.Cu) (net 6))
 (segment (start 64.77 38.1) (end 63.505199 39.364801) (width 0.25) (layer B.Cu) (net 6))
 (segment (start 43.18 41.91) (end 40.64 44.45) (width 0.25) (layer B.Cu) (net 6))
 (segment (start 40.64 62.23) (end 35.56 67.31) (width 0.25) (layer B.Cu) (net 6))
 (segment (start 40.64 44.45) (end 40.64 62.23) (width 0.25) (layer B.Cu) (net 6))
 (segment (start 44.45 60.96) (end 41.91 58.42) (width 0.25) (layer B.Cu) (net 7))
 (segment (start 41.91 46.594998) (end 41.91 57.28863) (width 0.25) (layer B.Cu) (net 7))
 (segment (start 47.719999 40.784999) (end 41.91 46.594998) (width 0.25) (layer B.Cu) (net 7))
 (segment (start 41.91 57.28863) (end 41.91 58.42) (width 0.25) (layer B.Cu) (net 7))
 (segment (start 64.625001 40.784999) (end 47.719999 40.784999) (width 0.25) (layer B.Cu) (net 7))
 (segment (start 67.31 38.1) (end 64.625001 40.784999) (width 0.25) (layer B.Cu) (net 7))
 (segment (start 53.34 45.72) (end 57.15 41.91) (width 0.25) (layer B.Cu) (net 8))
 (segment (start 44.45 45.72) (end 53.34 45.72) (width 0.25) (layer B.Cu) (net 8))
 (segment (start 66.04 41.91) (end 69.85 38.1) (width 0.25) (layer B.Cu) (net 8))
 (segment (start 57.15 41.91) (end 66.04 41.91) (width 0.25) (layer B.Cu) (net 8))
 (segment (start 67.31 58.42) (end 69.85 60.96) (width 0.25) (layer B.Cu) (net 9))
 (segment (start 71.450201 39.039799) (end 72.39 38.1) (width 0.25) (layer B.Cu) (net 9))
 (segment (start 71.055199 39.039799) (end 71.450201 39.039799) (width 0.25) (layer B.Cu) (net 9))
 (segment (start 67.31 42.784998) (end 71.055199 39.039799) (width 0.25) (layer B.Cu) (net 9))
 (segment (start 67.31 58.42) (end 67.31 42.784998) (width 0.25) (layer B.Cu) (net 9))
 (segment (start 70.649999 41.110001) (end 69.85 41.91) (width 0.25) (layer B.Cu) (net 10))
 (segment (start 71.484997 41.110001) (end 70.649999 41.110001) (width 0.25) (layer B.Cu) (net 10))
 (segment (start 73.555199 39.039799) (end 71.484997 41.110001) (width 0.25) (layer B.Cu) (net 10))
 (segment (start 73.990201 39.039799) (end 73.555199 39.039799) (width 0.25) (layer B.Cu) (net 10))
 (segment (start 74.93 38.1) (end 73.990201 39.039799) (width 0.25) (layer B.Cu) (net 10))
 (segment (start 69.85 41.91) (end 69.85 45.72) (width 0.25) (layer B.Cu) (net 10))
 (segment (start 95.25 60.96) (end 92.71 58.42) (width 0.25) (layer B.Cu) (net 11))
 (segment (start 92.71 58.42) (end 92.71 41.91) (width 0.25) (layer B.Cu) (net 11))
 (segment (start 77.47 38.1) (end 80.01 40.64) (width 0.25) (layer B.Cu) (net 11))
 (segment (start 91.44 40.64) (end 92.71 41.91) (width 0.25) (layer B.Cu) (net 11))
 (segment (start 80.01 40.64) (end 91.44 40.64) (width 0.25) (layer B.Cu) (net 11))
 (segment (start 95.25 45.72) (end 95.25 41.91) (width 0.25) (layer B.Cu) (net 12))
 (segment (start 92.71 39.37) (end 95.25 41.91) (width 0.25) (layer B.Cu) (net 12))
 (segment (start 80.01 38.1) (end 81.28 39.37) (width 0.25) (layer B.Cu) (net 12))
 (segment (start 81.28 39.37) (end 92.71 39.37) (width 0.25) (layer B.Cu) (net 12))
 (segment (start 102.87 48.26) (end 95.25 55.88) (width 0.25) (layer B.Cu) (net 19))
 (segment (start 109.22 48.26) (end 102.87 48.26) (width 0.25) (layer B.Cu) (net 19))
 (segment (start 101.6 62.23) (end 95.25 55.88) (width 0.25) (layer B.Cu) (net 19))
 (segment (start 101.6 64.77) (end 101.6 62.23) (width 0.25) (layer B.Cu) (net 19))
 (segment (start 109.22 73.66) (end 95.25 73.66) (width 0.25) (layer B.Cu) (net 18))
 (segment (start 95.25 73.66) (end 95.25 71.12) (width 0.25) (layer B.Cu) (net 18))
 (segment (start 69.85 55.88) (end 69.85 54.61) (width 0.25) (layer B.Cu) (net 17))
 (segment (start 76.2 48.26) (end 83.82 48.26) (width 0.25) (layer B.Cu) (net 17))
 (segment (start 69.85 54.61) (end 76.2 48.26) (width 0.25) (layer B.Cu) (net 17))
 (segment (start 76.2 62.23) (end 69.85 55.88) (width 0.25) (layer B.Cu) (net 17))
 (segment (start 76.2 64.77) (end 76.2 62.23) (width 0.25) (layer B.Cu) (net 17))
 (segment (start 83.82 73.66) (end 69.85 73.66) (width 0.25) (layer B.Cu) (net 16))
 (segment (start 69.85 73.66) (end 69.85 71.12) (width 0.25) (layer B.Cu) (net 16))
 (segment (start 52.07 48.26) (end 44.45 55.88) (width 0.25) (layer B.Cu) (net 15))
 (segment (start 58.42 48.26) (end 52.07 48.26) (width 0.25) (layer B.Cu) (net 15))
 (segment (start 50.8 62.23) (end 50.8 64.77) (width 0.25) (layer B.Cu) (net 15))
 (segment (start 44.45 55.88) (end 50.8 62.23) (width 0.25) (layer B.Cu) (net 15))
 (segment (start 58.42 73.66) (end 44.45 73.66) (width 0.25) (layer B.Cu) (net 14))
 (segment (start 44.45 73.66) (end 44.45 71.12) (width 0.25) (layer B.Cu) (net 14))
 (segment (start 34.29 90.17) (end 39.37 85.09) (width 0.25) (layer B.Cu) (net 2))
 (segment (start 33.02 73.66) (end 39.37 80.01) (width 0.25) (layer B.Cu) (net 2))
 (segment (start 39.37 80.01) (end 39.37 85.09) (width 0.25) (layer B.Cu) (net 2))
 (segment (start 26.67 67.31) (end 25.4 67.31) (width 0.25) (layer B.Cu) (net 2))
 (segment (start 33.02 73.66) (end 26.67 67.31) (width 0.25) (layer B.Cu) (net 2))
 (segment (start 30.48 34.29) (end 30.48 38.1) (width 0.25) (layer B.Cu) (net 13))
 (segment (start 30.48 45.72) (end 33.02 48.26) (width 0.25) (layer B.Cu) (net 13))
 (segment (start 30.48 38.1) (end 30.48 45.72) (width 0.25) (layer B.Cu) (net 13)))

